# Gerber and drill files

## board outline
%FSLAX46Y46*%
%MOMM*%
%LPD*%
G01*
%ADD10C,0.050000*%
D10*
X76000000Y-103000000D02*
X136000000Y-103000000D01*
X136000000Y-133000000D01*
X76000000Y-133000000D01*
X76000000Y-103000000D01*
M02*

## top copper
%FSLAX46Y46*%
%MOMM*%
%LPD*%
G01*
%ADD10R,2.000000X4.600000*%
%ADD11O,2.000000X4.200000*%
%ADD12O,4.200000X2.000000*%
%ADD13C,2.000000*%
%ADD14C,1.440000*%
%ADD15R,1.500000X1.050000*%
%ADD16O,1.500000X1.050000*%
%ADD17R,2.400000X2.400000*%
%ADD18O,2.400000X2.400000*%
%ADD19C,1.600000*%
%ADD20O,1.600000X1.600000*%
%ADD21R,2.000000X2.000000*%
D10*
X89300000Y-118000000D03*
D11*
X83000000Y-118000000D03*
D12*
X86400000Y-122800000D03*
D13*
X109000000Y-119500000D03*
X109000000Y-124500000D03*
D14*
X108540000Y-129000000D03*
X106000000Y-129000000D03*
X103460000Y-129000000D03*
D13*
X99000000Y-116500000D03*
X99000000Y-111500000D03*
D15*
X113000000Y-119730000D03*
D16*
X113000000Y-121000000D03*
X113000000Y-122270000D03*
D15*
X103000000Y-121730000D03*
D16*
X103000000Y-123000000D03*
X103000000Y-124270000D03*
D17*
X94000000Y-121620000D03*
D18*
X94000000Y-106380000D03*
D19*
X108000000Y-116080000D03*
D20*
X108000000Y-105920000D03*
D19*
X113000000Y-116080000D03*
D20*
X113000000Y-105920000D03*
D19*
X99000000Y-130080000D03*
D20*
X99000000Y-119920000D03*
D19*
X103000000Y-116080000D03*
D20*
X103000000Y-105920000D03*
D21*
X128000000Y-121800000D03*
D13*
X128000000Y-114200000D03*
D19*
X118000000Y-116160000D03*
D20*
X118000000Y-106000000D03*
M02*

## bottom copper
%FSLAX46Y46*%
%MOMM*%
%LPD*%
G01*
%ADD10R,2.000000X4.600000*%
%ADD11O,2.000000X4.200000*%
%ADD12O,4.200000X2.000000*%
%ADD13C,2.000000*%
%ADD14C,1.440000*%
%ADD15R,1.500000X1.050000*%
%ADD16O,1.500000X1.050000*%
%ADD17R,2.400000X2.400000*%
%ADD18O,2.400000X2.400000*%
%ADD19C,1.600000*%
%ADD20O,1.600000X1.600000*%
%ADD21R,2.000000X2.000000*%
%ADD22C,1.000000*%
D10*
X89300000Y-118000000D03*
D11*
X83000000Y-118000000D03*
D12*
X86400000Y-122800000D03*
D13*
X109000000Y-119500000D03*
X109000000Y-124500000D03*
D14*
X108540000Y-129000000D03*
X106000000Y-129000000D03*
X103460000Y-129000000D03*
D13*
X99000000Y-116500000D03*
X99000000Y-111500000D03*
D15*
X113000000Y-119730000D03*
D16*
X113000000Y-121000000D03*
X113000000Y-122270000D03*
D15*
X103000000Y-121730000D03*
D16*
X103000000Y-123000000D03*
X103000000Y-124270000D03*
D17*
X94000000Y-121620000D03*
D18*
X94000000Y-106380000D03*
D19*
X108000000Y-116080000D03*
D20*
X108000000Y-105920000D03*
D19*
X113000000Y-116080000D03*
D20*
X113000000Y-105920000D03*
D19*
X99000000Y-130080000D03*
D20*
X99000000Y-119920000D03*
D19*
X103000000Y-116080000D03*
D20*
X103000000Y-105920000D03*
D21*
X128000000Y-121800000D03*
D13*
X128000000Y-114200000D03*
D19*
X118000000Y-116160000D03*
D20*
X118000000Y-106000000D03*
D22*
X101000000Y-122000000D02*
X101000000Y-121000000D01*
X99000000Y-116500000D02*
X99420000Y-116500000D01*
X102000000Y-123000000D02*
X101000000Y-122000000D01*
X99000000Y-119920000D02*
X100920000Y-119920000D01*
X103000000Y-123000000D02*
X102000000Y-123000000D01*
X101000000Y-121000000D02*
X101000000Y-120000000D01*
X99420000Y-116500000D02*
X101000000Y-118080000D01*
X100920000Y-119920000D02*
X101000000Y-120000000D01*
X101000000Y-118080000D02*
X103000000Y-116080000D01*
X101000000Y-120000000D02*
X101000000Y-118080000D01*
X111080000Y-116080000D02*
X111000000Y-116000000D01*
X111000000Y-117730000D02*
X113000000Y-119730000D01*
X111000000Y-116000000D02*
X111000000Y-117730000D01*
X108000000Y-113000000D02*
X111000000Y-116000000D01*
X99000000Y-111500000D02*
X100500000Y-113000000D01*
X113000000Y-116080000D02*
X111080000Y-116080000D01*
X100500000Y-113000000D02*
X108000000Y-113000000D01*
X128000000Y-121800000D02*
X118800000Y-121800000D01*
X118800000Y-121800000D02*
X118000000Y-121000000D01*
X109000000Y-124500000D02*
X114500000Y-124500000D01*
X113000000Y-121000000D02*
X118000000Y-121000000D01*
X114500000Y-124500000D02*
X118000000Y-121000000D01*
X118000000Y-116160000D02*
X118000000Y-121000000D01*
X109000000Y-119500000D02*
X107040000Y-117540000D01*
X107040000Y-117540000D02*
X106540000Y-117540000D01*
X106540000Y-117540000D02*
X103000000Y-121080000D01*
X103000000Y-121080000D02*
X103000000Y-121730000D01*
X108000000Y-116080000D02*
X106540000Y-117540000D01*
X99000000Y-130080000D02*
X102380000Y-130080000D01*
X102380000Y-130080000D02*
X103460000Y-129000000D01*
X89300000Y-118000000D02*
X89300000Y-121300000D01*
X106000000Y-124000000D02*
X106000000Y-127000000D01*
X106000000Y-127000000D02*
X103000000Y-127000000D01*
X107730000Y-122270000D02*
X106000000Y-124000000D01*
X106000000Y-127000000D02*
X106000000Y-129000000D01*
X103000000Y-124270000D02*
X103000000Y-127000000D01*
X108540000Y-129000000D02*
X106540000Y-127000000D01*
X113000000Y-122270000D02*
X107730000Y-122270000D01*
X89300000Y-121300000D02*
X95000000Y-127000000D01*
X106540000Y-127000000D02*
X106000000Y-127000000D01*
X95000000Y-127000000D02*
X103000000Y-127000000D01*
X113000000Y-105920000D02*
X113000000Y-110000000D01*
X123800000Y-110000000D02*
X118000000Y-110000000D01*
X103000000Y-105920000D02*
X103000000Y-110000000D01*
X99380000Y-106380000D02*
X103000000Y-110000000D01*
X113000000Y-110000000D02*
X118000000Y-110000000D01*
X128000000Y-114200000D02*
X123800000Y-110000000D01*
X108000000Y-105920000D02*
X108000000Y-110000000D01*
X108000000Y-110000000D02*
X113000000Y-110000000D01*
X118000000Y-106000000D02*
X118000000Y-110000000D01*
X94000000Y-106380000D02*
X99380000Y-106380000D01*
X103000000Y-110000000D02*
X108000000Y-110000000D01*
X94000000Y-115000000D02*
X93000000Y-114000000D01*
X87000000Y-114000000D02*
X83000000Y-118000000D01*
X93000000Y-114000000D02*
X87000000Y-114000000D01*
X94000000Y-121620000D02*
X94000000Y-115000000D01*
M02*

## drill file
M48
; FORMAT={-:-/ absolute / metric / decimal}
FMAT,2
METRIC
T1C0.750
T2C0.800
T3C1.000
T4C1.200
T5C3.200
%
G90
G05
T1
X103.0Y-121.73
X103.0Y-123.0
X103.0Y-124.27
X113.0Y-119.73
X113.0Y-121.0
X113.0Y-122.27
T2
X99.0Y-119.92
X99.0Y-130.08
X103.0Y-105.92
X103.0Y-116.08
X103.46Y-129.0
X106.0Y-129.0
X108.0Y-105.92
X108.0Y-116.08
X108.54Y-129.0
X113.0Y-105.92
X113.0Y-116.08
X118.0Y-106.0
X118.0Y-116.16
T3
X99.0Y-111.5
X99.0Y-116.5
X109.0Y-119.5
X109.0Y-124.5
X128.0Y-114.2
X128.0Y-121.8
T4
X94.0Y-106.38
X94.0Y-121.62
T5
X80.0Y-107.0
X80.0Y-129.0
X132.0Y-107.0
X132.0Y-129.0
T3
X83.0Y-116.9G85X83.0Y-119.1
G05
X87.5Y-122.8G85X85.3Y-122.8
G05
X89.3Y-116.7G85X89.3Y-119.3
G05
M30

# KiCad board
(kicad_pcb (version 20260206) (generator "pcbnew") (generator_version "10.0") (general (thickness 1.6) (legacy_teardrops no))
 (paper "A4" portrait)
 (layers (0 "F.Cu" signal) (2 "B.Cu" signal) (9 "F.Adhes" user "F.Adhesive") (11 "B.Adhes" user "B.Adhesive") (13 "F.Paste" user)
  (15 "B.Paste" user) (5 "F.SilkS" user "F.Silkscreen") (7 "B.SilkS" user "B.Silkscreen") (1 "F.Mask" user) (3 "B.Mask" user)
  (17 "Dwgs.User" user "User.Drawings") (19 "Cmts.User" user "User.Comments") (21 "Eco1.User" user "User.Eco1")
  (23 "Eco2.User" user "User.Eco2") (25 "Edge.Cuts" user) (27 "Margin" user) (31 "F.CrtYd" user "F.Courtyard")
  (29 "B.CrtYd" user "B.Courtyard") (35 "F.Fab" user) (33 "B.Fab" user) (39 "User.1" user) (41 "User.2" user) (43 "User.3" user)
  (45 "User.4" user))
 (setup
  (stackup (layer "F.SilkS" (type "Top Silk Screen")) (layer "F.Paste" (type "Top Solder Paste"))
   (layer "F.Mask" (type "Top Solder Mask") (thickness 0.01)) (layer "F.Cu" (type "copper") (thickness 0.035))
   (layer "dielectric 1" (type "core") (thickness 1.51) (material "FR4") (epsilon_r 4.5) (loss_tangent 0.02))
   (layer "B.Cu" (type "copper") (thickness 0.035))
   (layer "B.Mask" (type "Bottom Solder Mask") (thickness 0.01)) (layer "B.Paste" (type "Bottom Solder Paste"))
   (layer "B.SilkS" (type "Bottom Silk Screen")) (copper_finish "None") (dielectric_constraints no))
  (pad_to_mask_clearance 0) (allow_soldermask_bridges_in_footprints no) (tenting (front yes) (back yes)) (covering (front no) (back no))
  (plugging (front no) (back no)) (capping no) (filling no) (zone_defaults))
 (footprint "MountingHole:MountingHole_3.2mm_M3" (layer "F.Cu") (at 80 129)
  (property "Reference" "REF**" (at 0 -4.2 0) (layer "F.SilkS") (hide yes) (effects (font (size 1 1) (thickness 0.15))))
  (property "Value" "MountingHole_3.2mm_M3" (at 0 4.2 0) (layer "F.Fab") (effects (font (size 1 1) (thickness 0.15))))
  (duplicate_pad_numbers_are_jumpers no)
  (pad "" np_thru_hole circle (at 0 0) (size 3.2 3.2) (drill 3.2) (layers "*.Cu" "*.Mask")))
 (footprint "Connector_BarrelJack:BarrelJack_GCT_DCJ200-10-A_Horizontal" (layer "F.Cu") (at 89.3 118 -90)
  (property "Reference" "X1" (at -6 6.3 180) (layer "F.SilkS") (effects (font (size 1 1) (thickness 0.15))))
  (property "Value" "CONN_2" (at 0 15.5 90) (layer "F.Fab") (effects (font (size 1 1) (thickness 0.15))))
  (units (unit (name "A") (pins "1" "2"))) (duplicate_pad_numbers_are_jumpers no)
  (pad "1" thru_hole rect (at 0 0 270) (size 4.6 2) (drill oval 3.6 1) (layers "*.Cu" "*.Mask") (remove_unused_layers no)
   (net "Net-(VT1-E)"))
  (pad "2" thru_hole oval (at 0 6.3 270) (size 4.2 2) (drill oval 3.2 1) (layers "*.Cu" "*.Mask") (remove_unused_layers no)
   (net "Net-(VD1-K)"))
  (pad "3" thru_hole oval (at 4.8 2.9 270) (size 2 4.2) (drill oval 1 3.2) (layers "*.Cu" "*.Mask") (remove_unused_layers no)))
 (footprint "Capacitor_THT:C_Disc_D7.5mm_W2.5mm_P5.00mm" (layer "F.Cu") (at 109 119.5 -90)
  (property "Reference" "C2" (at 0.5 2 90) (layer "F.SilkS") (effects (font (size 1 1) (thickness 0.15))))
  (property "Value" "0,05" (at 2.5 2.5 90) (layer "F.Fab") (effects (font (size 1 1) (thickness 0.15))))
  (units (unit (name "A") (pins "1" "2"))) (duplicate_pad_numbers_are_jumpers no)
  (pad "1" thru_hole circle (at 0 0 270) (size 2 2) (drill 1) (layers "*.Cu" "*.Mask") (remove_unused_layers no) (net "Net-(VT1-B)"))
  (pad "2" thru_hole circle (at 5 0 270) (size 2 2) (drill 1) (layers "*.Cu" "*.Mask") (remove_unused_layers no) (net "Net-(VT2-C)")))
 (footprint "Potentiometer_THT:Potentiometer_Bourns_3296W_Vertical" (layer "F.Cu") (at 108.54 129)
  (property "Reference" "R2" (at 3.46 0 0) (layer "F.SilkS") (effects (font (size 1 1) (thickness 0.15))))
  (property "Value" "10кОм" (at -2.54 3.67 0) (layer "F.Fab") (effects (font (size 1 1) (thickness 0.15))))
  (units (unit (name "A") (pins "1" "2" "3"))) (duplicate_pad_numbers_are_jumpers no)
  (pad "1" thru_hole circle (at 0 0) (size 1.44 1.44) (drill 0.8) (layers "*.Cu" "*.Mask") (remove_unused_layers no) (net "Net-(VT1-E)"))
  (pad "2" thru_hole circle (at -2.54 0) (size 1.44 1.44) (drill 0.8) (layers "*.Cu" "*.Mask") (remove_unused_layers no) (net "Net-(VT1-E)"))
  (pad "3" thru_hole circle (at -5.08 0) (size 1.44 1.44) (drill 0.8) (layers "*.Cu" "*.Mask") (remove_unused_layers no)
   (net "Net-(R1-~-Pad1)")))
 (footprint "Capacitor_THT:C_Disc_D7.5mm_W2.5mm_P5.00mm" (layer "F.Cu") (at 99 116.5 90)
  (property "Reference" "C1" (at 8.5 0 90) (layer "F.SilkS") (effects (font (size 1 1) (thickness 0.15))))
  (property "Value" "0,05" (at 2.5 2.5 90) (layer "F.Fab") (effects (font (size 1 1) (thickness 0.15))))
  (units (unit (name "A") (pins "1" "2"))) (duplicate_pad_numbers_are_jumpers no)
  (pad "1" thru_hole circle (at 0 0 90) (size 2 2) (drill 1) (layers "*.Cu" "*.Mask") (remove_unused_layers no) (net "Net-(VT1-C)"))
  (pad "2" thru_hole circle (at 5 0 90) (size 2 2) (drill 1) (layers "*.Cu" "*.Mask") (remove_unused_layers no) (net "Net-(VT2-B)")))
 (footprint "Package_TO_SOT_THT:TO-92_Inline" (layer "F.Cu") (at 113 119.73 -90)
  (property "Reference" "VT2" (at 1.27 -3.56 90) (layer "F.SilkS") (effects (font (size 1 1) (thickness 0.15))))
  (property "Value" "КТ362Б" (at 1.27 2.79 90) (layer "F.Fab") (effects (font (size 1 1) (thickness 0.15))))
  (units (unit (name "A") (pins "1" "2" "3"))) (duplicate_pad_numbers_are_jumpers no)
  (pad "1" thru_hole rect (at 0 0 270) (size 1.05 1.5) (drill 0.75) (layers "*.Cu" "*.Mask") (remove_unused_layers no) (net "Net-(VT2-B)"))
  (pad "2" thru_hole oval (at 1.27 0 270) (size 1.05 1.5) (drill 0.75) (layers "*.Cu" "*.Mask") (remove_unused_layers no)
   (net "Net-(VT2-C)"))
  (pad "3" thru_hole oval (at 2.54 0 270) (size 1.05 1.5) (drill 0.75) (layers "*.Cu" "*.Mask") (remove_unused_layers no)
   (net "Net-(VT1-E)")))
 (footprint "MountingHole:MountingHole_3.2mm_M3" (layer "F.Cu") (at 132 107)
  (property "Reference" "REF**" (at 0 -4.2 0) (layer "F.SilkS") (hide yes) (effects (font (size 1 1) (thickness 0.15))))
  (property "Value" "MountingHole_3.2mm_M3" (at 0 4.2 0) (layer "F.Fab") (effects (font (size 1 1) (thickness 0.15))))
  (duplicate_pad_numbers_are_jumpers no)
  (pad "" np_thru_hole circle (at 0 0) (size 3.2 3.2) (drill 3.2) (layers "*.Cu" "*.Mask")))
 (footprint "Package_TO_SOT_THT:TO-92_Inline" (layer "F.Cu") (at 103 121.73 -90)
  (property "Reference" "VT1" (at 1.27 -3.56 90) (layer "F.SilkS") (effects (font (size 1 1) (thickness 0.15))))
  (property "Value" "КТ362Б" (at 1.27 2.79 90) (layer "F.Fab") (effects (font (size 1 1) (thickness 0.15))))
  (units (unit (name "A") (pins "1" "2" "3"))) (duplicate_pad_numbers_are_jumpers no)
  (pad "1" thru_hole rect (at 0 0 270) (size 1.05 1.5) (drill 0.75) (layers "*.Cu" "*.Mask") (remove_unused_layers no) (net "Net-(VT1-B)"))
  (pad "2" thru_hole oval (at 1.27 0 270) (size 1.05 1.5) (drill 0.75) (layers "*.Cu" "*.Mask") (remove_unused_layers no)
   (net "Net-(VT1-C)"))
  (pad "3" thru_hole oval (at 2.54 0 270) (size 1.05 1.5) (drill 0.75) (layers "*.Cu" "*.Mask") (remove_unused_layers no)
   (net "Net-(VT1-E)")))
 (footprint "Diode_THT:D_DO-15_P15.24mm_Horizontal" (layer "F.Cu") (at 94 121.62 90)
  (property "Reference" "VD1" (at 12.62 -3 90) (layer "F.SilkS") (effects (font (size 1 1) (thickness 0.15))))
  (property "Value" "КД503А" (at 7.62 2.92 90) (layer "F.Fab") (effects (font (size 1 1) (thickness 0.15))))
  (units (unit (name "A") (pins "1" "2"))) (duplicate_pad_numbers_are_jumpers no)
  (pad "1" thru_hole rect (at 0 0 90) (size 2.4 2.4) (drill 1.2) (layers "*.Cu" "*.Mask") (remove_unused_layers no) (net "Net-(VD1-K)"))
  (pad "2" thru_hole oval (at 15.24 0 90) (size 2.4 2.4) (drill 1.2) (layers "*.Cu" "*.Mask") (remove_unused_layers no) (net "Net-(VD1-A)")))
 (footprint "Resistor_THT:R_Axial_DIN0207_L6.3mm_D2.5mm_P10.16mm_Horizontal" (layer "F.Cu") (at 108 116.08 90)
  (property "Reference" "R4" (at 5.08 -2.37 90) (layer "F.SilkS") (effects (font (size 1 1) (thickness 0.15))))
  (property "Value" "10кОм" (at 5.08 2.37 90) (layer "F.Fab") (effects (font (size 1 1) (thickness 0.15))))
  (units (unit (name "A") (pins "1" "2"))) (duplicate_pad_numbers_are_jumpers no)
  (pad "1" thru_hole circle (at 0 0 90) (size 1.6 1.6) (drill 0.8) (layers "*.Cu" "*.Mask") (remove_unused_layers no) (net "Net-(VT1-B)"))
  (pad "2" thru_hole oval (at 10.16 0 90) (size 1.6 1.6) (drill 0.8) (layers "*.Cu" "*.Mask") (remove_unused_layers no) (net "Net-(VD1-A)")))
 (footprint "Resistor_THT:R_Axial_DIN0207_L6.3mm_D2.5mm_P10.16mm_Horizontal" (layer "F.Cu") (at 113 116.08 90)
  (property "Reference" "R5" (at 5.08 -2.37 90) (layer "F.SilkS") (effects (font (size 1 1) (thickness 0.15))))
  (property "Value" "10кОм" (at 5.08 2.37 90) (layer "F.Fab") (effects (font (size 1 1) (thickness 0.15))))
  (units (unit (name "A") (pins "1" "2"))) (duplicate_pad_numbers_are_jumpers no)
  (pad "1" thru_hole circle (at 0 0 90) (size 1.6 1.6) (drill 0.8) (layers "*.Cu" "*.Mask") (remove_unused_layers no) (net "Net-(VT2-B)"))
  (pad "2" thru_hole oval (at 10.16 0 90) (size 1.6 1.6) (drill 0.8) (layers "*.Cu" "*.Mask") (remove_unused_layers no) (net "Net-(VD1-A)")))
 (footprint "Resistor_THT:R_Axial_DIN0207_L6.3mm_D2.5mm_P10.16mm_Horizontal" (layer "F.Cu") (at 99 130.08 90)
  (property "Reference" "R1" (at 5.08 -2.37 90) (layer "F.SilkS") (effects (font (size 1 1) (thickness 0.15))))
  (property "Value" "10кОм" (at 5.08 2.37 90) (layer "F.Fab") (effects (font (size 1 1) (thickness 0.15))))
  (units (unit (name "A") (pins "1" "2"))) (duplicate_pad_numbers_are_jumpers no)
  (pad "1" thru_hole circle (at 0 0 90) (size 1.6 1.6) (drill 0.8) (layers "*.Cu" "*.Mask") (remove_unused_layers no)
   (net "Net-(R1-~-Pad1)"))
  (pad "2" thru_hole oval (at 10.16 0 90) (size 1.6 1.6) (drill 0.8) (layers "*.Cu" "*.Mask") (remove_unused_layers no) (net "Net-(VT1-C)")))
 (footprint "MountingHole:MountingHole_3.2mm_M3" (layer "F.Cu") (at 80 107)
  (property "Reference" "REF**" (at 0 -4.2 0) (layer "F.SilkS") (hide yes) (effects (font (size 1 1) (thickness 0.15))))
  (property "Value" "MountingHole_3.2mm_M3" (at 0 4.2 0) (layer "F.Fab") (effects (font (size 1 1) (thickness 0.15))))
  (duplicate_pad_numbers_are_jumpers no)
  (pad "" np_thru_hole circle (at 0 0) (size 3.2 3.2) (drill 3.2) (layers "*.Cu" "*.Mask")))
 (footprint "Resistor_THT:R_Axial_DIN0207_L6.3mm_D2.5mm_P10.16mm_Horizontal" (layer "F.Cu") (at 103 116.08 90)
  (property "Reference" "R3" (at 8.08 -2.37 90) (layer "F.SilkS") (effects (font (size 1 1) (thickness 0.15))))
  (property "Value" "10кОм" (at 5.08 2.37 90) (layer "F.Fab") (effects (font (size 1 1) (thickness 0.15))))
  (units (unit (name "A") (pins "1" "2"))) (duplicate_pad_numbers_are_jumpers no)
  (pad "1" thru_hole circle (at 0 0 90) (size 1.6 1.6) (drill 0.8) (layers "*.Cu" "*.Mask") (remove_unused_layers no) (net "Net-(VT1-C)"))
  (pad "2" thru_hole oval (at 10.16 0 90) (size 1.6 1.6) (drill 0.8) (layers "*.Cu" "*.Mask") (remove_unused_layers no) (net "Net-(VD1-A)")))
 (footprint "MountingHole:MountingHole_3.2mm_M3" (layer "F.Cu") (at 132 129)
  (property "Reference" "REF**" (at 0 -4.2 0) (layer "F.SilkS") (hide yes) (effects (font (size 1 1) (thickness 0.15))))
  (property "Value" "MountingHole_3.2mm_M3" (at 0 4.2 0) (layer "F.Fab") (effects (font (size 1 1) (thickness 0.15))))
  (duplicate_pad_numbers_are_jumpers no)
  (pad "" np_thru_hole circle (at 0 0) (size 3.2 3.2) (drill 3.2) (layers "*.Cu" "*.Mask")))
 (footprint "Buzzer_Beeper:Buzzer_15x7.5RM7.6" (layer "F.Cu") (at 128 121.8 90)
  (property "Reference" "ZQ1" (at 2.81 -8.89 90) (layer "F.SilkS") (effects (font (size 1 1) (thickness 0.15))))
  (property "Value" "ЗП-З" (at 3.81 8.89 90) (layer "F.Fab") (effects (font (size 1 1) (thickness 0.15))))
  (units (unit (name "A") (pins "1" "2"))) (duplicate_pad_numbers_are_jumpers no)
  (pad "1" thru_hole rect (at 0 0 90) (size 2 2) (drill 1) (layers "*.Cu" "*.Mask") (remove_unused_layers no) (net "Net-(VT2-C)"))
  (pad "2" thru_hole circle (at 7.6 0 90) (size 2 2) (drill 1) (layers "*.Cu" "*.Mask") (remove_unused_layers no) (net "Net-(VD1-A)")))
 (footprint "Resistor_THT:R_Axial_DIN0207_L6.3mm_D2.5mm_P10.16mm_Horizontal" (layer "F.Cu") (at 118 116.16 90)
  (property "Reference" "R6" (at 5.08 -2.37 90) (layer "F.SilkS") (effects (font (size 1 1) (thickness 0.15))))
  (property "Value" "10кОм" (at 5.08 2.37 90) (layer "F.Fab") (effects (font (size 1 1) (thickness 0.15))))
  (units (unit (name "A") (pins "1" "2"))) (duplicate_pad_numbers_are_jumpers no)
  (pad "1" thru_hole circle (at 0 0 90) (size 1.6 1.6) (drill 0.8) (layers "*.Cu" "*.Mask") (remove_unused_layers no) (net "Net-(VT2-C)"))
  (pad "2" thru_hole oval (at 10.16 0 90) (size 1.6 1.6) (drill 0.8) (layers "*.Cu" "*.Mask") (remove_unused_layers no) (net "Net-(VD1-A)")))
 (gr_rect (start 76 103) (end 136 133) (stroke (width 0.05) (type default)) (fill no) (layer "Edge.Cuts"))
 (segment (start 101 122) (end 101 121) (width 1) (layer "B.Cu") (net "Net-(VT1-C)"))
 (segment (start 99 116.5) (end 99.42 116.5) (width 1) (layer "B.Cu") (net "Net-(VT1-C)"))
 (segment (start 102 123) (end 101 122) (width 1) (layer "B.Cu") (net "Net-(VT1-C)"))
 (segment (start 99 119.92) (end 100.92 119.92) (width 1) (layer "B.Cu") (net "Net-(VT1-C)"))
 (segment (start 103 123) (end 102 123) (width 1) (layer "B.Cu") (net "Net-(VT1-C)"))
 (segment (start 101 121) (end 101 120) (width 1) (layer "B.Cu") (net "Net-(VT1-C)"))
 (segment (start 99.42 116.5) (end 101 118.08) (width 1) (layer "B.Cu") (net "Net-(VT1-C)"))
 (segment (start 100.92 119.92) (end 101 120) (width 1) (layer "B.Cu") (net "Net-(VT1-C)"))
 (segment (start 101 118.08) (end 103 116.08) (width 1) (layer "B.Cu") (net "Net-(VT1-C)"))
 (segment (start 101 120) (end 101 118.08) (width 1) (layer "B.Cu") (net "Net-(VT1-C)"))
 (segment (start 111.08 116.08) (end 111 116) (width 1) (layer "B.Cu") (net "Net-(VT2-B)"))
 (segment (start 111 117.73) (end 113 119.73) (width 1) (layer "B.Cu") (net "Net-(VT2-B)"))
 (segment (start 111 116) (end 111 117.73) (width 1) (layer "B.Cu") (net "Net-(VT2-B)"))
 (segment (start 108 113) (end 111 116) (width 1) (layer "B.Cu") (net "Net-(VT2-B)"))
 (segment (start 99 111.5) (end 100.5 113) (width 1) (layer "B.Cu") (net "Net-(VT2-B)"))
 (segment (start 113 116.08) (end 111.08 116.08) (width 1) (layer "B.Cu") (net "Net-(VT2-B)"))
 (segment (start 100.5 113) (end 108 113) (width 1) (layer "B.Cu") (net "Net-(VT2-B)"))
 (segment (start 128 121.8) (end 118.8 121.8) (width 1) (layer "B.Cu") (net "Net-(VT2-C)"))
 (segment (start 118.8 121.8) (end 118 121) (width 1) (layer "B.Cu") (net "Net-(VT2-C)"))
 (segment (start 109 124.5) (end 114.5 124.5) (width 1) (layer "B.Cu") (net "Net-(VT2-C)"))
 (segment (start 113 121) (end 118 121) (width 1) (layer "B.Cu") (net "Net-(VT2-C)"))
 (segment (start 114.5 124.5) (end 118 121) (width 1) (layer "B.Cu") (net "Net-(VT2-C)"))
 (segment (start 118 116.16) (end 118 121) (width 1) (layer "B.Cu") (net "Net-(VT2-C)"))
 (segment (start 109 119.5) (end 107.04 117.54) (width 1) (layer "B.Cu") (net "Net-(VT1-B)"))
 (segment (start 107.04 117.54) (end 106.54 117.54) (width 1) (layer "B.Cu") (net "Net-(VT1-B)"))
 (segment (start 106.54 117.54) (end 103 121.08) (width 1) (layer "B.Cu") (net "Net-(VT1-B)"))
 (segment (start 103 121.08) (end 103 121.73) (width 1) (layer "B.Cu") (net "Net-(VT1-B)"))
 (segment (start 108 116.08) (end 106.54 117.54) (width 1) (layer "B.Cu") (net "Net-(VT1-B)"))
 (segment (start 99 130.08) (end 102.38 130.08) (width 1) (layer "B.Cu") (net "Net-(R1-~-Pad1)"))
 (segment (start 102.38 130.08) (end 103.46 129) (width 1) (layer "B.Cu") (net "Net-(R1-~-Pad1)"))
 (segment (start 89.3 118) (end 89.3 121.3) (width 1) (layer "B.Cu") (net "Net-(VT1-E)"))
 (segment (start 106 124) (end 106 127) (width 1) (layer "B.Cu") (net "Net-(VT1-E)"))
 (segment (start 106 127) (end 103 127) (width 1) (layer "B.Cu") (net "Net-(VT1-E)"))
 (segment (start 107.73 122.27) (end 106 124) (width 1) (layer "B.Cu") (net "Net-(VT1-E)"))
 (segment (start 106 127) (end 106 129) (width 1) (layer "B.Cu") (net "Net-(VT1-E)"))
 (segment (start 103 124.27) (end 103 127) (width 1) (layer "B.Cu") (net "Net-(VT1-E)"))
 (segment (start 108.54 129) (end 106.54 127) (width 1) (layer "B.Cu") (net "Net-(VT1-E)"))
 (segment (start 113 122.27) (end 107.73 122.27) (width 1) (layer "B.Cu") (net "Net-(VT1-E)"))
 (segment (start 89.3 121.3) (end 95 127) (width 1) (layer "B.Cu") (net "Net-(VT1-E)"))
 (segment (start 106.54 127) (end 106 127) (width 1) (layer "B.Cu") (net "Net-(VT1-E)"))
 (segment (start 95 127) (end 103 127) (width 1) (layer "B.Cu") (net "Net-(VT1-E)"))
 (segment (start 113 105.92) (end 113 110) (width 1) (layer "B.Cu") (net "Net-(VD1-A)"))
 (segment (start 123.8 110) (end 118 110) (width 1) (layer "B.Cu") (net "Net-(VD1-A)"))
 (segment (start 103 105.92) (end 103 110) (width 1) (layer "B.Cu") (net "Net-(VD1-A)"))
 (segment (start 99.38 106.38) (end 103 110) (width 1) (layer "B.Cu") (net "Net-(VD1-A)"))
 (segment (start 113 110) (end 118 110) (width 1) (layer "B.Cu") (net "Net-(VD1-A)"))
 (segment (start 128 114.2) (end 123.8 110) (width 1) (layer "B.Cu") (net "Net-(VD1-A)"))
 (segment (start 108 105.92) (end 108 110) (width 1) (layer "B.Cu") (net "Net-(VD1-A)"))
 (segment (start 108 110) (end 113 110) (width 1) (layer "B.Cu") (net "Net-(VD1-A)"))
 (segment (start 118 106) (end 118 110) (width 1) (layer "B.Cu") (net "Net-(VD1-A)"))
 (segment (start 94 106.38) (end 99.38 106.38) (width 1) (layer "B.Cu") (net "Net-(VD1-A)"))
 (segment (start 103 110) (end 108 110) (width 1) (layer "B.Cu") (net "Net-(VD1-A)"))
 (segment (start 94 115) (end 93 114) (width 1) (layer "B.Cu") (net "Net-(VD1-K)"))
 (segment (start 87 114) (end 83 118) (width 1) (layer "B.Cu") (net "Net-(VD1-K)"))
 (segment (start 93 114) (end 87 114) (width 1) (layer "B.Cu") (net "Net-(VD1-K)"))
 (segment (start 94 121.62) (end 94 115) (width 1) (layer "B.Cu") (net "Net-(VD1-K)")))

